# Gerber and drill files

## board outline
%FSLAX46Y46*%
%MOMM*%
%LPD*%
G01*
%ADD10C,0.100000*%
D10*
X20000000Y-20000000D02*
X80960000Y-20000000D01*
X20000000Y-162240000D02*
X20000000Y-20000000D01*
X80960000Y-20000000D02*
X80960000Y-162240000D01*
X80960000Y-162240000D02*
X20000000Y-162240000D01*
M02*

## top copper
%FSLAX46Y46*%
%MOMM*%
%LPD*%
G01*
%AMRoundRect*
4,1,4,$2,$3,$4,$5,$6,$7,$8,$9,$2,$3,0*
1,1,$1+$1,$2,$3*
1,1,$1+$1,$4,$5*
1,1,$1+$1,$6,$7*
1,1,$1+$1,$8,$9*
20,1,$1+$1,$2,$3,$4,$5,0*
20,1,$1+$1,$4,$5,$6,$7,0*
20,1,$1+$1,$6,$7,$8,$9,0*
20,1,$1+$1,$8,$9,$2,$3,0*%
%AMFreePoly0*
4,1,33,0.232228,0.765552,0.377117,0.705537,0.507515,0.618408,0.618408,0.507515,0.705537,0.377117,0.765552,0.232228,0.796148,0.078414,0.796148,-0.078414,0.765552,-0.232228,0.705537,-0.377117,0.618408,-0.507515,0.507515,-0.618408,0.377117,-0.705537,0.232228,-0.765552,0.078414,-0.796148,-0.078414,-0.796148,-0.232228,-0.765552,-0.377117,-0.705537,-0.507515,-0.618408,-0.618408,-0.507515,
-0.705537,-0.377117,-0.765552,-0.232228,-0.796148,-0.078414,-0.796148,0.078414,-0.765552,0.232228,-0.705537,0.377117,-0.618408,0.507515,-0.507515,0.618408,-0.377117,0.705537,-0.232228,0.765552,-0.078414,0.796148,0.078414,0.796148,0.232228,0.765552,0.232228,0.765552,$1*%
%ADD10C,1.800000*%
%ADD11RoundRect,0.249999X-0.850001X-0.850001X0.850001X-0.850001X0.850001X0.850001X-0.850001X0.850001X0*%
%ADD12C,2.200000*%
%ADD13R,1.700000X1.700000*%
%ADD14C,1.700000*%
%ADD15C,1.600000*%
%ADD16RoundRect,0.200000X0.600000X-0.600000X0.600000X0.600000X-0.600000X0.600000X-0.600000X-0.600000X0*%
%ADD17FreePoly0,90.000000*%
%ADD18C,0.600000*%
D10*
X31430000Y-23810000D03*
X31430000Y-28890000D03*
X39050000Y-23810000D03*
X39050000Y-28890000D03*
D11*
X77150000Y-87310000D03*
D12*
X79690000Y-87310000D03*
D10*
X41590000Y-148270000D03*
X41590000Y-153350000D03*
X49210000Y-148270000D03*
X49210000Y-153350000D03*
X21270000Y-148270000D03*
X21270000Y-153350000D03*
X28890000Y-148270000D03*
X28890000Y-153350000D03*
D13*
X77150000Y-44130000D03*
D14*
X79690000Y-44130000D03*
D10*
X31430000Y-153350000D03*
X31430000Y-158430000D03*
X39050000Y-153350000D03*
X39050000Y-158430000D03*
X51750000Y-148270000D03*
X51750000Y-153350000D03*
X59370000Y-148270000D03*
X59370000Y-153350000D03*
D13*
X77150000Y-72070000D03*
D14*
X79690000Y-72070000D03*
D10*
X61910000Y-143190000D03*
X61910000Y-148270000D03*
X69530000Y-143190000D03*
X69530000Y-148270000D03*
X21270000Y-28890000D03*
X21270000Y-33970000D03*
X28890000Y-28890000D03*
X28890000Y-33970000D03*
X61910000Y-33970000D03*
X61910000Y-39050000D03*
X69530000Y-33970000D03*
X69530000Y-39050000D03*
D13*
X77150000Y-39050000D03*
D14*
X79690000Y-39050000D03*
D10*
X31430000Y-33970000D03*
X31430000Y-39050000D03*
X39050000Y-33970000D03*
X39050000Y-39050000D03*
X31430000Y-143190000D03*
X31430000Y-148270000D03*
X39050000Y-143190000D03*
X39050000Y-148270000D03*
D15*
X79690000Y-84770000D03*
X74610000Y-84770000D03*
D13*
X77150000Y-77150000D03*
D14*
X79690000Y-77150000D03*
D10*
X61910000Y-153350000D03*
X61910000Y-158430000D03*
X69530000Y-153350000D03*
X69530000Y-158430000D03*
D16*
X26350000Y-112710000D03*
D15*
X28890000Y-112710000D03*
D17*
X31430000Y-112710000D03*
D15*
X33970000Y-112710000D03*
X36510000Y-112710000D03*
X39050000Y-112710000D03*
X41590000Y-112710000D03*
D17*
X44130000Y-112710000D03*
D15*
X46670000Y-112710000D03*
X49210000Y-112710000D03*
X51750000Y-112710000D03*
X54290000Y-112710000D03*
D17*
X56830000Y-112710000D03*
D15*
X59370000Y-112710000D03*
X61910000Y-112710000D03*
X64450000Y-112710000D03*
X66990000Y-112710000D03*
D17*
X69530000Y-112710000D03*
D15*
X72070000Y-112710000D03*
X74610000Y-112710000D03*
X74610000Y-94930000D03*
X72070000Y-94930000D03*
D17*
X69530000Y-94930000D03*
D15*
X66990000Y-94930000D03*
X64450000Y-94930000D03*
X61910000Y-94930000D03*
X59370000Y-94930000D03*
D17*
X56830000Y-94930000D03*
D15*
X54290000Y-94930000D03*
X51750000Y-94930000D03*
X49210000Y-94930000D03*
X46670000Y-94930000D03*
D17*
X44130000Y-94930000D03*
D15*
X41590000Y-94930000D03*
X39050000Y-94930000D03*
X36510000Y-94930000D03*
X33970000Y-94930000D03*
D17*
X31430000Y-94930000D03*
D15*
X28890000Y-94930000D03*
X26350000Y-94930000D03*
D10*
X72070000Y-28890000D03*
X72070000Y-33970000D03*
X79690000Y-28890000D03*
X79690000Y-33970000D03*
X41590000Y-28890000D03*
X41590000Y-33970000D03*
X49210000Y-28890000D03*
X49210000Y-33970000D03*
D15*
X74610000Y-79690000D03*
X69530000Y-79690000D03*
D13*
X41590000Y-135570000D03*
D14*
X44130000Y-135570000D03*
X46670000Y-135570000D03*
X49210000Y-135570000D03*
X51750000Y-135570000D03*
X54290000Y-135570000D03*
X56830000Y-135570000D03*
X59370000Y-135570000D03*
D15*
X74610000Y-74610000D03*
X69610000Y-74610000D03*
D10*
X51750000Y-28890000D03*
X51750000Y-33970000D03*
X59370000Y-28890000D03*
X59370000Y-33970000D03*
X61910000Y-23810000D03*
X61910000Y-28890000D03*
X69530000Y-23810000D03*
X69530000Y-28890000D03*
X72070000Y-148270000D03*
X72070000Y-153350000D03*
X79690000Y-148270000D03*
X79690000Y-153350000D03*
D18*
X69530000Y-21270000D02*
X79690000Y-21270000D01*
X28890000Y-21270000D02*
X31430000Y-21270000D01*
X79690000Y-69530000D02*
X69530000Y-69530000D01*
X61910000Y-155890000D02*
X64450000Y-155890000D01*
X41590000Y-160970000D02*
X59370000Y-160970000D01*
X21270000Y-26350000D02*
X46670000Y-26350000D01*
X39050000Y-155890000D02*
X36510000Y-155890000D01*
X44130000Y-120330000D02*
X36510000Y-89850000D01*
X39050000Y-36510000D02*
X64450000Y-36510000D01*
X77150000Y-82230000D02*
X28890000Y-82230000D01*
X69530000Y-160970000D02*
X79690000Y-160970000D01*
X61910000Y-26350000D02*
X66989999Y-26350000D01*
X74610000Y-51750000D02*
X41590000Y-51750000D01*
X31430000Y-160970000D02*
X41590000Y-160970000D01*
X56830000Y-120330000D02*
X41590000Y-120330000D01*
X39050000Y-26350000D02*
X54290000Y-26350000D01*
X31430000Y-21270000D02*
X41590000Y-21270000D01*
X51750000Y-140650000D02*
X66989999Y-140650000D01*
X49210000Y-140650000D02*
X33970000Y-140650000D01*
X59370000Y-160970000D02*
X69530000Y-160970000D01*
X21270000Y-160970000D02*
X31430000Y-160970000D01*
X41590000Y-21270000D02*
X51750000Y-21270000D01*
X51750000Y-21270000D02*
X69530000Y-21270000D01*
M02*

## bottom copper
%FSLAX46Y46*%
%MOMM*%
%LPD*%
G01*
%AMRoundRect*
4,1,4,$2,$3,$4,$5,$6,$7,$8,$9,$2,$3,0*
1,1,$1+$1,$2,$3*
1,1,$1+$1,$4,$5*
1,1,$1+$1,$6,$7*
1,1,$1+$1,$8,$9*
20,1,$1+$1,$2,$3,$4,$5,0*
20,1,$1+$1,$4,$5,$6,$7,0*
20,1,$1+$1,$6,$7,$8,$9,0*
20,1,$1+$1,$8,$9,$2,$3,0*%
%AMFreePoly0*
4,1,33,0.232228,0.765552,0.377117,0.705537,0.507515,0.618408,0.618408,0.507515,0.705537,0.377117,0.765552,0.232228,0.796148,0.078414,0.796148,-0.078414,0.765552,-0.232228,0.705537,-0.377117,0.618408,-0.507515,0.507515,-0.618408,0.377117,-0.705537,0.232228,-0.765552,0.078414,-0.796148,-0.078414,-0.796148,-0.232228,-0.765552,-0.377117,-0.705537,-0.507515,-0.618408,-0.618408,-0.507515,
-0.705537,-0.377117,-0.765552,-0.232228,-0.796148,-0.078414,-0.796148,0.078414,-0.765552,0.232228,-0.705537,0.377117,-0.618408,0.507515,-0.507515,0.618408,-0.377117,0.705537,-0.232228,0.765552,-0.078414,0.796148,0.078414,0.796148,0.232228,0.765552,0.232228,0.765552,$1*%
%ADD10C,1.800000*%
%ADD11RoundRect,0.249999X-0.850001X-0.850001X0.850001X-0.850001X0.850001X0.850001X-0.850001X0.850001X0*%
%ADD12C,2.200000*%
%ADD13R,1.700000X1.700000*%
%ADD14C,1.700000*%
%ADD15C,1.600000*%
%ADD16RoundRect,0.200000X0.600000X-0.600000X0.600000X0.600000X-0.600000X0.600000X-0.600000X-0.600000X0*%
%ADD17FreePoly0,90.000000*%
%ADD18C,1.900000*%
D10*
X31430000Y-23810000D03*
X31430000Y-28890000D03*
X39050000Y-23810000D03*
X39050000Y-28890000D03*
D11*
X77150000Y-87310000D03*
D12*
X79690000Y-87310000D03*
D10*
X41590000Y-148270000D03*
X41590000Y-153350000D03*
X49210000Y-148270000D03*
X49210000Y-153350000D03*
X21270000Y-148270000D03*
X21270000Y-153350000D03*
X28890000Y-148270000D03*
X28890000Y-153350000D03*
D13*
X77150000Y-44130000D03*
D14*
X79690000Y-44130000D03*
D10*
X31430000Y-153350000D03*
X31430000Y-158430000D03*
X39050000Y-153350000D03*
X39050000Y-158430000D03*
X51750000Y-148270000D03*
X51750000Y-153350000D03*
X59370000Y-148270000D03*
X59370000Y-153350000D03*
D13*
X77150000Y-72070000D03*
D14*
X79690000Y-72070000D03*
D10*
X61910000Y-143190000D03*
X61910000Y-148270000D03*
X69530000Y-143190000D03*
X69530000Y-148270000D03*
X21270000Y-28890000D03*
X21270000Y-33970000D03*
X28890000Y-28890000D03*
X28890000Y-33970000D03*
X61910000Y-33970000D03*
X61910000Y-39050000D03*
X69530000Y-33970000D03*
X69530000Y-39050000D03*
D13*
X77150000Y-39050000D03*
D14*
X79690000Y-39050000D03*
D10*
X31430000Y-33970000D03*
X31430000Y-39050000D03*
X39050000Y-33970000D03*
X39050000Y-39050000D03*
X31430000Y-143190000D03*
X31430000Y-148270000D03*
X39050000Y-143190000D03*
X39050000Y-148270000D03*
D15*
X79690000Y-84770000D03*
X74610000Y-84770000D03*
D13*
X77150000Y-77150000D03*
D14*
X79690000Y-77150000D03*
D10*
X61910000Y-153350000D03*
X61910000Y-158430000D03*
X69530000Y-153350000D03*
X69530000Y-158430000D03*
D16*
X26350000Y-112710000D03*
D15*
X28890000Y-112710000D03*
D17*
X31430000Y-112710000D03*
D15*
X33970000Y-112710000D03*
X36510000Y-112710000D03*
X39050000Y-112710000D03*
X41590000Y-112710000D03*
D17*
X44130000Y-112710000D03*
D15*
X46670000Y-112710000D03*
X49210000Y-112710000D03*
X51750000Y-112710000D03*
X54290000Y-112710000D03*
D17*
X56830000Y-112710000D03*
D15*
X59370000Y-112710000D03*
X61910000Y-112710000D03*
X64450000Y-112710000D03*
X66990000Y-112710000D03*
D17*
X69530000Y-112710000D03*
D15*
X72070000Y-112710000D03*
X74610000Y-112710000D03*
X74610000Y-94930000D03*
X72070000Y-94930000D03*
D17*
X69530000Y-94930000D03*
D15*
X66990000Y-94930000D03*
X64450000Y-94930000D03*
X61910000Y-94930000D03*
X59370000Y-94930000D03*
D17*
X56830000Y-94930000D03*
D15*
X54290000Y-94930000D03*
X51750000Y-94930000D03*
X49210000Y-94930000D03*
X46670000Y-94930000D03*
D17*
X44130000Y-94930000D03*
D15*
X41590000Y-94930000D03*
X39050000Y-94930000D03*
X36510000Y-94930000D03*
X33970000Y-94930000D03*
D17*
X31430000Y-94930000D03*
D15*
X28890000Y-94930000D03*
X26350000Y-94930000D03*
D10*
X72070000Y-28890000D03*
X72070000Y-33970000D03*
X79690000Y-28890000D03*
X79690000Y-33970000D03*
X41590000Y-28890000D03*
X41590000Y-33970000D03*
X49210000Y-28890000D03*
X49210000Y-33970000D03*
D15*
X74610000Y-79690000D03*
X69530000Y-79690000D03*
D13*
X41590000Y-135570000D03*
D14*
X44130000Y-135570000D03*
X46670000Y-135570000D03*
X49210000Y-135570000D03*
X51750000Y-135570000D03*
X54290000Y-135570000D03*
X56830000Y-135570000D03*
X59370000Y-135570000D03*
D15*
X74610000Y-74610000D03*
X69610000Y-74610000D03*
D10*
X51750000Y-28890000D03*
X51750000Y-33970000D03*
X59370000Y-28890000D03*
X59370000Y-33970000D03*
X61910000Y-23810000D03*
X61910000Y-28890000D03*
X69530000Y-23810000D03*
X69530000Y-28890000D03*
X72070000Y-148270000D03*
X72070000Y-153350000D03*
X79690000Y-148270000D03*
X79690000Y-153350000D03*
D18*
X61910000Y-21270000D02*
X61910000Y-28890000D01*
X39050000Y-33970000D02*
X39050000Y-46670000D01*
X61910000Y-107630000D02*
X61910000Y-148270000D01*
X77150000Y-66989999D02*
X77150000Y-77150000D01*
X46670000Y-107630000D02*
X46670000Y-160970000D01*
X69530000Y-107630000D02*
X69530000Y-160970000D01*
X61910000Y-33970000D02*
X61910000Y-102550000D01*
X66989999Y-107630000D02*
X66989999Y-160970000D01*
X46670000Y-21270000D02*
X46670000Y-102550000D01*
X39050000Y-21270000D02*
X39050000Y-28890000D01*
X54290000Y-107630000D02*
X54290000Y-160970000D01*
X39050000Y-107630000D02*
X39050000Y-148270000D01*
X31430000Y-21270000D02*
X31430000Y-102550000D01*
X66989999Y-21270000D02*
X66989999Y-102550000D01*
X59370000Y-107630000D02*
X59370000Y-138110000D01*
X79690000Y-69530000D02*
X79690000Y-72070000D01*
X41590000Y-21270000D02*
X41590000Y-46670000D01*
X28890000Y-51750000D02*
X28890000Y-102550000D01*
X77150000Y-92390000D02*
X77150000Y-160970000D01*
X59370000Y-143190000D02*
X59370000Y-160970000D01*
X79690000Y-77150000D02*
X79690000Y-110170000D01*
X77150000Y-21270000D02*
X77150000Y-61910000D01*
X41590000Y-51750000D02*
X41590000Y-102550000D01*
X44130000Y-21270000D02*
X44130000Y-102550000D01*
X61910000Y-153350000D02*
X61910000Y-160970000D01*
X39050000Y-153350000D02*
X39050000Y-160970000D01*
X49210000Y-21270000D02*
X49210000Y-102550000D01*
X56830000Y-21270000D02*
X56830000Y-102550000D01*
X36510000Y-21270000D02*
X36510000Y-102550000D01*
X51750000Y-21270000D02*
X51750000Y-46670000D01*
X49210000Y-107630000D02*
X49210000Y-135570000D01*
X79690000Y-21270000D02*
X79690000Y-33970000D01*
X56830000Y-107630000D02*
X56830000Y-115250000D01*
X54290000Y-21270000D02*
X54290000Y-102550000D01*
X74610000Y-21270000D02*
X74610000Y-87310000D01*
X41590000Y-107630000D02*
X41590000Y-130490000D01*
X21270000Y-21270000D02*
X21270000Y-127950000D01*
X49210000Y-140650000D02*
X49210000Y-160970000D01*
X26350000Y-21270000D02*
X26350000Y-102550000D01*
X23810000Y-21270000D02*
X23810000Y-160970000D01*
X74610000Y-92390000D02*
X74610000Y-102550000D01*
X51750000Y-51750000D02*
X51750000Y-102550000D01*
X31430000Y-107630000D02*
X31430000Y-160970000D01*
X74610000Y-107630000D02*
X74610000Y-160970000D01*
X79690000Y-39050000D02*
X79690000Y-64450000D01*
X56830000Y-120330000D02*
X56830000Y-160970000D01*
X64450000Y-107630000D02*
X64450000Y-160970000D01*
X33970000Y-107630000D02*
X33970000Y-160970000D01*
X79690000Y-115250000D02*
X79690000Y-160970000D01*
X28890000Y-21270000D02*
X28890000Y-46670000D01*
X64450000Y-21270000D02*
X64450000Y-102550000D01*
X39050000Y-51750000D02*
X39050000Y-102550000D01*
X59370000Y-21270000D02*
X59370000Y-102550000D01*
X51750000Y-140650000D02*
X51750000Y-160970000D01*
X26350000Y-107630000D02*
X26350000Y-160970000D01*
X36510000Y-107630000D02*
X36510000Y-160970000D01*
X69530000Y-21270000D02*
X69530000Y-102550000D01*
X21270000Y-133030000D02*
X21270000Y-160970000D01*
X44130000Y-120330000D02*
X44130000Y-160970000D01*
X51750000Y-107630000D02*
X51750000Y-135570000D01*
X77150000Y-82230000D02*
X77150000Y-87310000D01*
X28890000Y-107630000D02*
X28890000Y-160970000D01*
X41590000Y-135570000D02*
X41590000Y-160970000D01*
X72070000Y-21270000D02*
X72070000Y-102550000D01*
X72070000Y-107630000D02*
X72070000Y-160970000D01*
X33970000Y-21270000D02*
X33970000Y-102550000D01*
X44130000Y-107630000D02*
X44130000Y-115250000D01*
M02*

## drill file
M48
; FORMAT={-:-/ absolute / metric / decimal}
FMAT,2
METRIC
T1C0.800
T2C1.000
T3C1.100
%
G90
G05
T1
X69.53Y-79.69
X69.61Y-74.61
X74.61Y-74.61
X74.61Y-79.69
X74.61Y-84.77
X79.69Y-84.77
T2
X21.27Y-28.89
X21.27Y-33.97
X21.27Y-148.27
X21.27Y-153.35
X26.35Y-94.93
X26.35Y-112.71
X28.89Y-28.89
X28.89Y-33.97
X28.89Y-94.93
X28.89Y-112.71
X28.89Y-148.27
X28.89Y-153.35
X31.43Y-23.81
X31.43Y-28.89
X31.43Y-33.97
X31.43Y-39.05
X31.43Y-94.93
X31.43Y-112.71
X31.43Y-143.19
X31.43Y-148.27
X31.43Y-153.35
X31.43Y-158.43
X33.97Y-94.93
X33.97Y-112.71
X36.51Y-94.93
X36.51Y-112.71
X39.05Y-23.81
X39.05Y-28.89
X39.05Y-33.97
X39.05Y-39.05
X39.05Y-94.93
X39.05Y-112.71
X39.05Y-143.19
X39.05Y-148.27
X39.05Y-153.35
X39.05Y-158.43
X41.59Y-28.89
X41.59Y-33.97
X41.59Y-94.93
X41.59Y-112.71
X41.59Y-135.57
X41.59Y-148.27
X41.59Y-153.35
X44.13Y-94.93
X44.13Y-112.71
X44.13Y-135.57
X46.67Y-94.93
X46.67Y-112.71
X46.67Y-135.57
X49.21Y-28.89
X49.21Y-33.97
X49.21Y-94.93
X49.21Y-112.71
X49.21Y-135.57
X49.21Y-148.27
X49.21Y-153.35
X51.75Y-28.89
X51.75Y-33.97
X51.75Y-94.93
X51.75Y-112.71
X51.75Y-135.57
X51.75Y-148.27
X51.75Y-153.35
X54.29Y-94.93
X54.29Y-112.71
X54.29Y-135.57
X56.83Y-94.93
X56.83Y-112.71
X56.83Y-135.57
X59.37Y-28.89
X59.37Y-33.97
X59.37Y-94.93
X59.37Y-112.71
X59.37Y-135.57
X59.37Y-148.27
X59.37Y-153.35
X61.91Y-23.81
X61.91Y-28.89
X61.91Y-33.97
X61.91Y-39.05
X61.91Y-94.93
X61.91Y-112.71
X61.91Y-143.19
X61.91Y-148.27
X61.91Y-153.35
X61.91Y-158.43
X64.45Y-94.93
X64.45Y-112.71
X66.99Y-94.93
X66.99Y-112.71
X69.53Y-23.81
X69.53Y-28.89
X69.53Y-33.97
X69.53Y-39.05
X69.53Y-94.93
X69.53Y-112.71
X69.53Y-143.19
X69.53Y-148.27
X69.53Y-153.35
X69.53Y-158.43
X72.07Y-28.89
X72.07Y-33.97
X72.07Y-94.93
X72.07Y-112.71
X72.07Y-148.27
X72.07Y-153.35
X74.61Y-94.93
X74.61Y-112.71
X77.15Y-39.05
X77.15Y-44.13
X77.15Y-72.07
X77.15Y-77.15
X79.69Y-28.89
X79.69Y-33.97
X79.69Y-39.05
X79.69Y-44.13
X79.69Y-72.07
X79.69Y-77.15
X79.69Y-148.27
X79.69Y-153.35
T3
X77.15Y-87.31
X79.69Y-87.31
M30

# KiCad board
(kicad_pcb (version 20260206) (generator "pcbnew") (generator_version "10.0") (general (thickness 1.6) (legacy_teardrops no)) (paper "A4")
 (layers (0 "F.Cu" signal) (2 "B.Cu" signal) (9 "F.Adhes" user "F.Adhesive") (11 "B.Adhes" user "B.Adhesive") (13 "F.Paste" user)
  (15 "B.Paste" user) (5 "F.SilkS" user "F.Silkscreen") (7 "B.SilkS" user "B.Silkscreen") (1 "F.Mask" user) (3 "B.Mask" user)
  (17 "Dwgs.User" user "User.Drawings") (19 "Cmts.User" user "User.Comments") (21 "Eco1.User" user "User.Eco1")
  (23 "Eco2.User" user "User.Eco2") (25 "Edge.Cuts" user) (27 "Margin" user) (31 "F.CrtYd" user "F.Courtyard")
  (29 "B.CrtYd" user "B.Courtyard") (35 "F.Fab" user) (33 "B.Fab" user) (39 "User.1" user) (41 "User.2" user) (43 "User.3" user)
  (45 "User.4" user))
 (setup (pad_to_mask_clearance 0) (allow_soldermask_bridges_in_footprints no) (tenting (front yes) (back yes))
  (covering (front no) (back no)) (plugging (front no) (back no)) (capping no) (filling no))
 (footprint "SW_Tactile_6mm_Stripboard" (layer "F.Cu") (at 31.43 23.81)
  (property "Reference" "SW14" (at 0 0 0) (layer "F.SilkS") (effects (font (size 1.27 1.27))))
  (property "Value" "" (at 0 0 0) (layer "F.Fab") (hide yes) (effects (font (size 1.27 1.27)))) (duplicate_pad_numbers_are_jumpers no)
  (pad "1" thru_hole circle (at 0 0) (size 1.8 1.8) (drill 1) (layers "*.Cu" "*.Mask") (remove_unused_layers no))
  (pad "1" thru_hole circle (at 0 5.08) (size 1.8 1.8) (drill 1) (layers "*.Cu" "*.Mask") (remove_unused_layers no))
  (pad "2" thru_hole circle (at 7.62 0) (size 1.8 1.8) (drill 1) (layers "*.Cu" "*.Mask") (remove_unused_layers no))
  (pad "2" thru_hole circle (at 7.62 5.08) (size 1.8 1.8) (drill 1) (layers "*.Cu" "*.Mask") (remove_unused_layers no)))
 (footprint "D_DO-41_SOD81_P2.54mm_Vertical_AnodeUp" (layer "F.Cu") (at 77.15 87.31)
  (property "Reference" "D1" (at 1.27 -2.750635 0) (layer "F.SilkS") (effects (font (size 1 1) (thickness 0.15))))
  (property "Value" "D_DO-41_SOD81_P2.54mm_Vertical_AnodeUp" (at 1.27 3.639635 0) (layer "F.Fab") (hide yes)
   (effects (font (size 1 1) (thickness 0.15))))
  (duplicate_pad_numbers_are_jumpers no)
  (pad "1" thru_hole roundrect (at 0 0) (size 2.2 2.2) (drill 1.1) (layers "*.Cu" "*.Mask") (remove_unused_layers no)
   (roundrect_rratio 0.113636))
  (pad "2" thru_hole circle (at 2.54 0) (size 2.2 2.2) (drill 1.1) (layers "*.Cu" "*.Mask") (remove_unused_layers no)))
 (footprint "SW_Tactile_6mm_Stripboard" (layer "F.Cu") (at 41.59 148.27)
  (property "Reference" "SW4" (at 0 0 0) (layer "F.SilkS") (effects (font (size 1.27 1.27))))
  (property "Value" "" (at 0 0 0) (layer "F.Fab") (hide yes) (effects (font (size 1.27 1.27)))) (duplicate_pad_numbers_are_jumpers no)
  (pad "1" thru_hole circle (at 0 0) (size 1.8 1.8) (drill 1) (layers "*.Cu" "*.Mask") (remove_unused_layers no))
  (pad "1" thru_hole circle (at 0 5.08) (size 1.8 1.8) (drill 1) (layers "*.Cu" "*.Mask") (remove_unused_layers no))
  (pad "2" thru_hole circle (at 7.62 0) (size 1.8 1.8) (drill 1) (layers "*.Cu" "*.Mask") (remove_unused_layers no))
  (pad "2" thru_hole circle (at 7.62 5.08) (size 1.8 1.8) (drill 1) (layers "*.Cu" "*.Mask") (remove_unused_layers no)))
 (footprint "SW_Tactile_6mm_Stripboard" (layer "F.Cu") (at 21.27 148.27)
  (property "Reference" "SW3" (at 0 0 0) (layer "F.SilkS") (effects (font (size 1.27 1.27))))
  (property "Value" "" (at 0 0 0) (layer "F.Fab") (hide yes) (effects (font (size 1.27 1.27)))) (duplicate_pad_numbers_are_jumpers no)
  (pad "1" thru_hole circle (at 0 0) (size 1.8 1.8) (drill 1) (layers "*.Cu" "*.Mask") (remove_unused_layers no))
  (pad "1" thru_hole circle (at 0 5.08) (size 1.8 1.8) (drill 1) (layers "*.Cu" "*.Mask") (remove_unused_layers no))
  (pad "2" thru_hole circle (at 7.62 0) (size 1.8 1.8) (drill 1) (layers "*.Cu" "*.Mask") (remove_unused_layers no))
  (pad "2" thru_hole circle (at 7.62 5.08) (size 1.8 1.8) (drill 1) (layers "*.Cu" "*.Mask") (remove_unused_layers no)))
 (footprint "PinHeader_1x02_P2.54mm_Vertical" (layer "F.Cu") (at 77.15 44.13 90)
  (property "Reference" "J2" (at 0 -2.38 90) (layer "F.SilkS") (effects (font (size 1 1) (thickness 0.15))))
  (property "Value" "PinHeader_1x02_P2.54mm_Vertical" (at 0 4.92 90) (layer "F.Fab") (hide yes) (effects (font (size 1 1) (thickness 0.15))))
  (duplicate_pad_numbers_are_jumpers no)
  (pad "1" thru_hole rect (at 0 0 90) (size 1.7 1.7) (drill 1) (layers "*.Cu" "*.Mask") (remove_unused_layers no))
  (pad "2" thru_hole circle (at 0 2.54 90) (size 1.7 1.7) (drill 1) (layers "*.Cu" "*.Mask") (remove_unused_layers no)))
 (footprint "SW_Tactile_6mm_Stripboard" (layer "F.Cu") (at 31.43 153.35)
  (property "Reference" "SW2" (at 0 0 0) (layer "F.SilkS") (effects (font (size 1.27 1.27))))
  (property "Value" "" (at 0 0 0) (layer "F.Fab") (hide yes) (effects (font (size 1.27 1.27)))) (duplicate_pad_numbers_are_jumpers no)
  (pad "1" thru_hole circle (at 0 0) (size 1.8 1.8) (drill 1) (layers "*.Cu" "*.Mask") (remove_unused_layers no))
  (pad "1" thru_hole circle (at 0 5.08) (size 1.8 1.8) (drill 1) (layers "*.Cu" "*.Mask") (remove_unused_layers no))
  (pad "2" thru_hole circle (at 7.62 0) (size 1.8 1.8) (drill 1) (layers "*.Cu" "*.Mask") (remove_unused_layers no))
  (pad "2" thru_hole circle (at 7.62 5.08) (size 1.8 1.8) (drill 1) (layers "*.Cu" "*.Mask") (remove_unused_layers no)))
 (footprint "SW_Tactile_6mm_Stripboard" (layer "F.Cu") (at 51.75 148.27)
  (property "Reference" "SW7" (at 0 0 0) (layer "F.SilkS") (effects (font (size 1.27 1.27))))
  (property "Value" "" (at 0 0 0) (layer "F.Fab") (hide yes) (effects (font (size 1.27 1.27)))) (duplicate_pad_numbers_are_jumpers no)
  (pad "1" thru_hole circle (at 0 0) (size 1.8 1.8) (drill 1) (layers "*.Cu" "*.Mask") (remove_unused_layers no))
  (pad "1" thru_hole circle (at 0 5.08) (size 1.8 1.8) (drill 1) (layers "*.Cu" "*.Mask") (remove_unused_layers no))
  (pad "2" thru_hole circle (at 7.62 0) (size 1.8 1.8) (drill 1) (layers "*.Cu" "*.Mask") (remove_unused_layers no))
  (pad "2" thru_hole circle (at 7.62 5.08) (size 1.8 1.8) (drill 1) (layers "*.Cu" "*.Mask") (remove_unused_layers no)))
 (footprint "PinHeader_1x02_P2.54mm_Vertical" (layer "F.Cu") (at 77.15 72.07 90)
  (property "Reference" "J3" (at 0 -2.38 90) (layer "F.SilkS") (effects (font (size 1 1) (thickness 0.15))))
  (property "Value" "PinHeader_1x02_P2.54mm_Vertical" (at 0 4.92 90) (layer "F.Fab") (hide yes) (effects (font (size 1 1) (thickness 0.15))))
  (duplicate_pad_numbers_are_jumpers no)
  (pad "1" thru_hole rect (at 0 0 90) (size 1.7 1.7) (drill 1) (layers "*.Cu" "*.Mask") (remove_unused_layers no))
  (pad "2" thru_hole circle (at 0 2.54 90) (size 1.7 1.7) (drill 1) (layers "*.Cu" "*.Mask") (remove_unused_layers no)))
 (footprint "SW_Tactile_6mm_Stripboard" (layer "F.Cu") (at 61.91 143.19)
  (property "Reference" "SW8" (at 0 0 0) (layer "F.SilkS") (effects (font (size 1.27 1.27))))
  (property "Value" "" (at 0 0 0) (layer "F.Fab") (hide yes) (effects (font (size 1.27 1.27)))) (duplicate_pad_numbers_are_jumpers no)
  (pad "1" thru_hole circle (at 0 0) (size 1.8 1.8) (drill 1) (layers "*.Cu" "*.Mask") (remove_unused_layers no))
  (pad "1" thru_hole circle (at 0 5.08) (size 1.8 1.8) (drill 1) (layers "*.Cu" "*.Mask") (remove_unused_layers no))
  (pad "2" thru_hole circle (at 7.62 0) (size 1.8 1.8) (drill 1) (layers "*.Cu" "*.Mask") (remove_unused_layers no))
  (pad "2" thru_hole circle (at 7.62 5.08) (size 1.8 1.8) (drill 1) (layers "*.Cu" "*.Mask") (remove_unused_layers no)))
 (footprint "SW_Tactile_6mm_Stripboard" (layer "F.Cu") (at 21.27 28.89)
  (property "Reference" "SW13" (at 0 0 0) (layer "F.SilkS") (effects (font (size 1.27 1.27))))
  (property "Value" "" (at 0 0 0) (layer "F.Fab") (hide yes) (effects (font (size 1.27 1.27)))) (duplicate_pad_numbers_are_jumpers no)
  (pad "1" thru_hole circle (at 0 0) (size 1.8 1.8) (drill 1) (layers "*.Cu" "*.Mask") (remove_unused_layers no))
  (pad "1" thru_hole circle (at 0 5.08) (size 1.8 1.8) (drill 1) (layers "*.Cu" "*.Mask") (remove_unused_layers no))
  (pad "2" thru_hole circle (at 7.62 0) (size 1.8 1.8) (drill 1) (layers "*.Cu" "*.Mask") (remove_unused_layers no))
  (pad "2" thru_hole circle (at 7.62 5.08) (size 1.8 1.8) (drill 1) (layers "*.Cu" "*.Mask") (remove_unused_layers no)))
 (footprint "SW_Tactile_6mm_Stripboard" (layer "F.Cu") (at 61.91 33.97)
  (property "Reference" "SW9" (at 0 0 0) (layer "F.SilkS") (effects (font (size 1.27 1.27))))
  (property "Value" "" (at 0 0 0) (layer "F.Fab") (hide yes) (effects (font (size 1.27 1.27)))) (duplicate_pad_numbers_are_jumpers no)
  (pad "1" thru_hole circle (at 0 0) (size 1.8 1.8) (drill 1) (layers "*.Cu" "*.Mask") (remove_unused_layers no))
  (pad "1" thru_hole circle (at 0 5.08) (size 1.8 1.8) (drill 1) (layers "*.Cu" "*.Mask") (remove_unused_layers no))
  (pad "2" thru_hole circle (at 7.62 0) (size 1.8 1.8) (drill 1) (layers "*.Cu" "*.Mask") (remove_unused_layers no))
  (pad "2" thru_hole circle (at 7.62 5.08) (size 1.8 1.8) (drill 1) (layers "*.Cu" "*.Mask") (remove_unused_layers no)))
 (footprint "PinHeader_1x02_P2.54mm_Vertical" (layer "F.Cu") (at 77.15 39.05 90)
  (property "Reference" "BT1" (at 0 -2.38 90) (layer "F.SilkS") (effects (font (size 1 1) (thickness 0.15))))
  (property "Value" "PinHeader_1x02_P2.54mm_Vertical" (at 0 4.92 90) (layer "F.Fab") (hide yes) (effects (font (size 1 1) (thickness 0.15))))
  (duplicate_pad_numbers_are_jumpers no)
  (pad "1" thru_hole rect (at 0 0 90) (size 1.7 1.7) (drill 1) (layers "*.Cu" "*.Mask") (remove_unused_layers no))
  (pad "2" thru_hole circle (at 0 2.54 90) (size 1.7 1.7) (drill 1) (layers "*.Cu" "*.Mask") (remove_unused_layers no)))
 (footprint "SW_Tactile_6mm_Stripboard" (layer "F.Cu") (at 31.43 33.97)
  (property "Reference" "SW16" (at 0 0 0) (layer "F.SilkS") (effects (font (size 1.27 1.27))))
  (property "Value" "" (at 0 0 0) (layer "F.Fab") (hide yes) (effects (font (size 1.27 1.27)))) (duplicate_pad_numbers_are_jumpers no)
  (pad "1" thru_hole circle (at 0 0) (size 1.8 1.8) (drill 1) (layers "*.Cu" "*.Mask") (remove_unused_layers no))
  (pad "1" thru_hole circle (at 0 5.08) (size 1.8 1.8) (drill 1) (layers "*.Cu" "*.Mask") (remove_unused_layers no))
  (pad "2" thru_hole circle (at 7.62 0) (size 1.8 1.8) (drill 1) (layers "*.Cu" "*.Mask") (remove_unused_layers no))
  (pad "2" thru_hole circle (at 7.62 5.08) (size 1.8 1.8) (drill 1) (layers "*.Cu" "*.Mask") (remove_unused_layers no)))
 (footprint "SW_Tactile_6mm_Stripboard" (layer "F.Cu") (at 31.43 143.19)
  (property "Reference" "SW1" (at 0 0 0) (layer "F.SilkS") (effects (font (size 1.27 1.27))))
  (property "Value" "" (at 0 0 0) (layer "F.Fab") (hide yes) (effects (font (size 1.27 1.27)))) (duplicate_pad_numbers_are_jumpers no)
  (pad "1" thru_hole circle (at 0 0) (size 1.8 1.8) (drill 1) (layers "*.Cu" "*.Mask") (remove_unused_layers no))
  (pad "1" thru_hole circle (at 0 5.08) (size 1.8 1.8) (drill 1) (layers "*.Cu" "*.Mask") (remove_unused_layers no))
  (pad "2" thru_hole circle (at 7.62 0) (size 1.8 1.8) (drill 1) (layers "*.Cu" "*.Mask") (remove_unused_layers no))
  (pad "2" thru_hole circle (at 7.62 5.08) (size 1.8 1.8) (drill 1) (layers "*.Cu" "*.Mask") (remove_unused_layers no)))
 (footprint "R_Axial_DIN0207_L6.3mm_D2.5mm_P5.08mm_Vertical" (layer "F.Cu") (at 79.69 84.77 180)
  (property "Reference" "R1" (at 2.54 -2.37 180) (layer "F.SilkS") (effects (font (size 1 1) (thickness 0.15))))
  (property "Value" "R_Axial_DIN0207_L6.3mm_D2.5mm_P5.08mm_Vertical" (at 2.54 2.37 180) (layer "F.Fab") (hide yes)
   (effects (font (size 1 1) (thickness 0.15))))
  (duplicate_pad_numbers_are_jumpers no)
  (pad "1" thru_hole circle (at 0 0 180) (size 1.6 1.6) (drill 0.8) (layers "*.Cu" "*.Mask") (remove_unused_layers no))
  (pad "2" thru_hole circle (at 5.08 0 180) (size 1.6 1.6) (drill 0.8) (layers "*.Cu" "*.Mask") (remove_unused_layers no)))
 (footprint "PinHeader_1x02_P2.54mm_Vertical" (layer "F.Cu") (at 77.15 77.15 90)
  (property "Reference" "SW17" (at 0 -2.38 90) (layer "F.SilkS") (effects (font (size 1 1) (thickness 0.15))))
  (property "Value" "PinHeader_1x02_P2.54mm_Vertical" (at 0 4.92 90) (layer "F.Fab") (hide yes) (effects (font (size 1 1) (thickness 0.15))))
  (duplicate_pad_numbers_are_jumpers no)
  (pad "1" thru_hole rect (at 0 0 90) (size 1.7 1.7) (drill 1) (layers "*.Cu" "*.Mask") (remove_unused_layers no))
  (pad "2" thru_hole circle (at 0 2.54 90) (size 1.7 1.7) (drill 1) (layers "*.Cu" "*.Mask") (remove_unused_layers no)))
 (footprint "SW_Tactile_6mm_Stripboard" (layer "F.Cu") (at 61.91 153.35)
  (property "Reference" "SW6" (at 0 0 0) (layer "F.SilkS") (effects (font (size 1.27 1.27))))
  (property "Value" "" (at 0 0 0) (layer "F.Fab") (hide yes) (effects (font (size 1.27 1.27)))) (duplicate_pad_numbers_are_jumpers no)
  (pad "1" thru_hole circle (at 0 0) (size 1.8 1.8) (drill 1) (layers "*.Cu" "*.Mask") (remove_unused_layers no))
  (pad "1" thru_hole circle (at 0 5.08) (size 1.8 1.8) (drill 1) (layers "*.Cu" "*.Mask") (remove_unused_layers no))
  (pad "2" thru_hole circle (at 7.62 0) (size 1.8 1.8) (drill 1) (layers "*.Cu" "*.Mask") (remove_unused_layers no))
  (pad "2" thru_hole circle (at 7.62 5.08) (size 1.8 1.8) (drill 1) (layers "*.Cu" "*.Mask") (remove_unused_layers no)))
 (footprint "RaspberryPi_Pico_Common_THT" (layer "F.Cu") (at 26.35 112.71 90)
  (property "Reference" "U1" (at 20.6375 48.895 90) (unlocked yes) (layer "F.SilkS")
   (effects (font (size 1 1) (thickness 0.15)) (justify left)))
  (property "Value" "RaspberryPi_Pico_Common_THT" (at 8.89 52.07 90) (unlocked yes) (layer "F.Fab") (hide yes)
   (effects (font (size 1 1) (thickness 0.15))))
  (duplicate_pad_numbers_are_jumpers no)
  (pad "1" thru_hole roundrect (at 0 0 90) (size 1.6 1.6) (drill 1) (layers "*.Cu" "*.Mask") (remove_unused_layers no)
   (roundrect_rratio 0.125))
  (pad "2" thru_hole circle (at 0 2.54 90) (size 1.6 1.6) (drill 1) (layers "*.Cu" "*.Mask") (remove_unused_layers no))
  (pad "3" thru_hole custom (at 0 5.08 90) (size 1.6 1.6) (drill 1) (layers "*.Cu" "*.Mask") (remove_unused_layers no)
   (options (clearance outline) (anchor circle)) (primitives))
  (pad "4" thru_hole circle (at 0 7.62 90) (size 1.6 1.6) (drill 1) (layers "*.Cu" "*.Mask") (remove_unused_layers no))
  (pad "5" thru_hole circle (at 0 10.16 90) (size 1.6 1.6) (drill 1) (layers "*.Cu" "*.Mask") (remove_unused_layers no))
  (pad "6" thru_hole circle (at 0 12.7 90) (size 1.6 1.6) (drill 1) (layers "*.Cu" "*.Mask") (remove_unused_layers no))
  (pad "7" thru_hole circle (at 0 15.24 90) (size 1.6 1.6) (drill 1) (layers "*.Cu" "*.Mask") (remove_unused_layers no))
  (pad "8" thru_hole custom (at 0 17.78 90) (size 1.6 1.6) (drill 1) (layers "*.Cu" "*.Mask") (remove_unused_layers no)
   (options (clearance outline) (anchor circle)) (primitives))
  (pad "9" thru_hole circle (at 0 20.32 90) (size 1.6 1.6) (drill 1) (layers "*.Cu" "*.Mask") (remove_unused_layers no))
  (pad "10" thru_hole circle (at 0 22.86 90) (size 1.6 1.6) (drill 1) (layers "*.Cu" "*.Mask") (remove_unused_layers no))
  (pad "11" thru_hole circle (at 0 25.4 90) (size 1.6 1.6) (drill 1) (layers "*.Cu" "*.Mask") (remove_unused_layers no))
  (pad "12" thru_hole circle (at 0 27.94 90) (size 1.6 1.6) (drill 1) (layers "*.Cu" "*.Mask") (remove_unused_layers no))
  (pad "13" thru_hole custom (at 0 30.48 90) (size 1.6 1.6) (drill 1) (layers "*.Cu" "*.Mask") (remove_unused_layers no)
   (options (clearance outline) (anchor circle)) (primitives))
  (pad "14" thru_hole circle (at 0 33.02 90) (size 1.6 1.6) (drill 1) (layers "*.Cu" "*.Mask") (remove_unused_layers no))
  (pad "15" thru_hole circle (at 0 35.56 90) (size 1.6 1.6) (drill 1) (layers "*.Cu" "*.Mask") (remove_unused_layers no))
  (pad "16" thru_hole circle (at 0 38.1 90) (size 1.6 1.6) (drill 1) (layers "*.Cu" "*.Mask") (remove_unused_layers no))
  (pad "17" thru_hole circle (at 0 40.64 90) (size 1.6 1.6) (drill 1) (layers "*.Cu" "*.Mask") (remove_unused_layers no))
  (pad "18" thru_hole custom (at 0 43.18 90) (size 1.6 1.6) (drill 1) (layers "*.Cu" "*.Mask") (remove_unused_layers no)
   (options (clearance outline) (anchor circle)) (primitives))
  (pad "19" thru_hole circle (at 0 45.72 90) (size 1.6 1.6) (drill 1) (layers "*.Cu" "*.Mask") (remove_unused_layers no))
  (pad "20" thru_hole circle (at 0 48.26 90) (size 1.6 1.6) (drill 1) (layers "*.Cu" "*.Mask") (remove_unused_layers no))
  (pad "21" thru_hole circle (at 17.78 48.26 90) (size 1.6 1.6) (drill 1) (layers "*.Cu" "*.Mask") (remove_unused_layers no))
  (pad "22" thru_hole circle (at 17.78 45.72 90) (size 1.6 1.6) (drill 1) (layers "*.Cu" "*.Mask") (remove_unused_layers no))
  (pad "23" thru_hole custom (at 17.78 43.18 90) (size 1.6 1.6) (drill 1) (layers "*.Cu" "*.Mask") (remove_unused_layers no)
   (options (clearance outline) (anchor circle)) (primitives))
  (pad "24" thru_hole circle (at 17.78 40.64 90) (size 1.6 1.6) (drill 1) (layers "*.Cu" "*.Mask") (remove_unused_layers no))
  (pad "25" thru_hole circle (at 17.78 38.1 90) (size 1.6 1.6) (drill 1) (layers "*.Cu" "*.Mask") (remove_unused_layers no))
  (pad "26" thru_hole circle (at 17.78 35.56 90) (size 1.6 1.6) (drill 1) (layers "*.Cu" "*.Mask") (remove_unused_layers no))
  (pad "27" thru_hole circle (at 17.78 33.02 90) (size 1.6 1.6) (drill 1) (layers "*.Cu" "*.Mask") (remove_unused_layers no))
  (pad "28" thru_hole custom (at 17.78 30.48 90) (size 1.6 1.6) (drill 1) (layers "*.Cu" "*.Mask") (remove_unused_layers no)
   (options (clearance outline) (anchor circle)) (primitives))
  (pad "29" thru_hole circle (at 17.78 27.94 90) (size 1.6 1.6) (drill 1) (layers "*.Cu" "*.Mask") (remove_unused_layers no))
  (pad "30" thru_hole circle (at 17.78 25.4 90) (size 1.6 1.6) (drill 1) (layers "*.Cu" "*.Mask") (remove_unused_layers no))
  (pad "31" thru_hole circle (at 17.78 22.86 90) (size 1.6 1.6) (drill 1) (layers "*.Cu" "*.Mask") (remove_unused_layers no))
  (pad "32" thru_hole circle (at 17.78 20.32 90) (size 1.6 1.6) (drill 1) (layers "*.Cu" "*.Mask") (remove_unused_layers no))
  (pad "33" thru_hole custom (at 17.78 17.78 90) (size 1.6 1.6) (drill 1) (layers "*.Cu" "*.Mask") (remove_unused_layers no)
   (options (clearance outline) (anchor circle)) (primitives))
  (pad "34" thru_hole circle (at 17.78 15.24 90) (size 1.6 1.6) (drill 1) (layers "*.Cu" "*.Mask") (remove_unused_layers no))
  (pad "35" thru_hole circle (at 17.78 12.7 90) (size 1.6 1.6) (drill 1) (layers "*.Cu" "*.Mask") (remove_unused_layers no))
  (pad "36" thru_hole circle (at 17.78 10.16 90) (size 1.6 1.6) (drill 1) (layers "*.Cu" "*.Mask") (remove_unused_layers no))
  (pad "37" thru_hole circle (at 17.78 7.62 90) (size 1.6 1.6) (drill 1) (layers "*.Cu" "*.Mask") (remove_unused_layers no))
  (pad "38" thru_hole custom (at 17.78 5.08 90) (size 1.6 1.6) (drill 1) (layers "*.Cu" "*.Mask") (remove_unused_layers no)
   (options (clearance outline) (anchor circle)) (primitives))
  (pad "39" thru_hole circle (at 17.78 2.54 90) (size 1.6 1.6) (drill 1) (layers "*.Cu" "*.Mask") (remove_unused_layers no))
  (pad "40" thru_hole circle (at 17.78 0 90) (size 1.6 1.6) (drill 1) (layers "*.Cu" "*.Mask") (remove_unused_layers no))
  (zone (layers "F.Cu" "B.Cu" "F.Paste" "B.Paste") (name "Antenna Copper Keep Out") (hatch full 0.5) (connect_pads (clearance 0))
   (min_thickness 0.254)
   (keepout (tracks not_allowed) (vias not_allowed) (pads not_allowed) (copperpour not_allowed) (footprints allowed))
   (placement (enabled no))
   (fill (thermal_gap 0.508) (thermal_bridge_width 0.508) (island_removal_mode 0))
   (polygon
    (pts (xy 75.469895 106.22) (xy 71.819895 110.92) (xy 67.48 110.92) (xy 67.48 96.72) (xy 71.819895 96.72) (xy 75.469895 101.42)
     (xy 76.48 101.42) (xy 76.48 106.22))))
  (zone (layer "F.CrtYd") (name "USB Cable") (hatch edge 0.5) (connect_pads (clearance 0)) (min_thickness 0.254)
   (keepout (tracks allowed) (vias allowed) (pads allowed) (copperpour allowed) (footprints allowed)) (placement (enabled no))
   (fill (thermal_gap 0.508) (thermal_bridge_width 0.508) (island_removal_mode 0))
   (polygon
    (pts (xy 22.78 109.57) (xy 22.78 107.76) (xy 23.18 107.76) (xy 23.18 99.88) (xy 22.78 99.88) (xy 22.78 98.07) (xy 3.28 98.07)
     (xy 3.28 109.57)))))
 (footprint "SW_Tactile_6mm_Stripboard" (layer "F.Cu") (at 72.07 28.89)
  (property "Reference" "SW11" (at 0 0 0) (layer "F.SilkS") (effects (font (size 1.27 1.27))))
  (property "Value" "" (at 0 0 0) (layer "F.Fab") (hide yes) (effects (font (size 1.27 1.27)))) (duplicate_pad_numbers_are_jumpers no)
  (pad "1" thru_hole circle (at 0 0) (size 1.8 1.8) (drill 1) (layers "*.Cu" "*.Mask") (remove_unused_layers no))
  (pad "1" thru_hole circle (at 0 5.08) (size 1.8 1.8) (drill 1) (layers "*.Cu" "*.Mask") (remove_unused_layers no))
  (pad "2" thru_hole circle (at 7.62 0) (size 1.8 1.8) (drill 1) (layers "*.Cu" "*.Mask") (remove_unused_layers no))
  (pad "2" thru_hole circle (at 7.62 5.08) (size 1.8 1.8) (drill 1) (layers "*.Cu" "*.Mask") (remove_unused_layers no)))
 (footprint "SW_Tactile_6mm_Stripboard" (layer "F.Cu") (at 41.59 28.89)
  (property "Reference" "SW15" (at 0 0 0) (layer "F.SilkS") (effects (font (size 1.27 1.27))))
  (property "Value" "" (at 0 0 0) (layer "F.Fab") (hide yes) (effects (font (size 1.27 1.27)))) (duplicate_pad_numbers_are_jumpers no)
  (pad "1" thru_hole circle (at 0 0) (size 1.8 1.8) (drill 1) (layers "*.Cu" "*.Mask") (remove_unused_layers no))
  (pad "1" thru_hole circle (at 0 5.08) (size 1.8 1.8) (drill 1) (layers "*.Cu" "*.Mask") (remove_unused_layers no))
  (pad "2" thru_hole circle (at 7.62 0) (size 1.8 1.8) (drill 1) (layers "*.Cu" "*.Mask") (remove_unused_layers no))
  (pad "2" thru_hole circle (at 7.62 5.08) (size 1.8 1.8) (drill 1) (layers "*.Cu" "*.Mask") (remove_unused_layers no)))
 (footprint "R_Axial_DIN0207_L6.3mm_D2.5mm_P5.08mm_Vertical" (layer "F.Cu") (at 74.61 79.69 180)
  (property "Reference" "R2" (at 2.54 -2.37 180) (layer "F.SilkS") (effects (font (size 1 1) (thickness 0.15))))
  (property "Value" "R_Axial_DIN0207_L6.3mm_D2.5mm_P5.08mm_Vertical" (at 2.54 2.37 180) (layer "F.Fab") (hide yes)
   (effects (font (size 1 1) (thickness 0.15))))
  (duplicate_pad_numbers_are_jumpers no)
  (pad "1" thru_hole circle (at 0 0 180) (size 1.6 1.6) (drill 0.8) (layers "*.Cu" "*.Mask") (remove_unused_layers no))
  (pad "2" thru_hole circle (at 5.08 0 180) (size 1.6 1.6) (drill 0.8) (layers "*.Cu" "*.Mask") (remove_unused_layers no)))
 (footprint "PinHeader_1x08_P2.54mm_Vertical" (layer "F.Cu") (at 41.59 135.57 90)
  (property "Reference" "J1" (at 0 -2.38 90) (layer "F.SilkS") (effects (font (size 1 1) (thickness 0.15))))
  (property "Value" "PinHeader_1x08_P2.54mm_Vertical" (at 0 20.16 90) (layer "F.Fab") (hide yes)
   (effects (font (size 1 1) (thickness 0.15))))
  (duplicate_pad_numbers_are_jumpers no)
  (pad "1" thru_hole rect (at 0 0 90) (size 1.7 1.7) (drill 1) (layers "*.Cu" "*.Mask") (remove_unused_layers no))
  (pad "2" thru_hole circle (at 0 2.54 90) (size 1.7 1.7) (drill 1) (layers "*.Cu" "*.Mask") (remove_unused_layers no))
  (pad "3" thru_hole circle (at 0 5.08 90) (size 1.7 1.7) (drill 1) (layers "*.Cu" "*.Mask") (remove_unused_layers no))
  (pad "4" thru_hole circle (at 0 7.62 90) (size 1.7 1.7) (drill 1) (layers "*.Cu" "*.Mask") (remove_unused_layers no))
  (pad "5" thru_hole circle (at 0 10.16 90) (size 1.7 1.7) (drill 1) (layers "*.Cu" "*.Mask") (remove_unused_layers no))
  (pad "6" thru_hole circle (at 0 12.7 90) (size 1.7 1.7) (drill 1) (layers "*.Cu" "*.Mask") (remove_unused_layers no))
  (pad "7" thru_hole circle (at 0 15.24 90) (size 1.7 1.7) (drill 1) (layers "*.Cu" "*.Mask") (remove_unused_layers no))
  (pad "8" thru_hole circle (at 0 17.78 90) (size 1.7 1.7) (drill 1) (layers "*.Cu" "*.Mask") (remove_unused_layers no)))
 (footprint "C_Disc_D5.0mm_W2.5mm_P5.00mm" (layer "F.Cu") (at 74.61 74.61 180)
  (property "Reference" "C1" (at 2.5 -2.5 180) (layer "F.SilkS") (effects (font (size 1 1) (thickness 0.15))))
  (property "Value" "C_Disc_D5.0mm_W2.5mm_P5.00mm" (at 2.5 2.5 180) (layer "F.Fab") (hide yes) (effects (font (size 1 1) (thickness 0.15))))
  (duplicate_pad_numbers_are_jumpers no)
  (pad "1" thru_hole circle (at 0 0 180) (size 1.6 1.6) (drill 0.8) (layers "*.Cu" "*.Mask") (remove_unused_layers no))
  (pad "2" thru_hole circle (at 5 0 180) (size 1.6 1.6) (drill 0.8) (layers "*.Cu" "*.Mask") (remove_unused_layers no)))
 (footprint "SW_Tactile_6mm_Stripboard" (layer "F.Cu") (at 51.75 28.89)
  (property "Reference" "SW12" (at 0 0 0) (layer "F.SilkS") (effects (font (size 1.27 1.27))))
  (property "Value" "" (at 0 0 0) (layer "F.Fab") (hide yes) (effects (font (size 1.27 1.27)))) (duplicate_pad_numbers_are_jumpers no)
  (pad "1" thru_hole circle (at 0 0) (size 1.8 1.8) (drill 1) (layers "*.Cu" "*.Mask") (remove_unused_layers no))
  (pad "1" thru_hole circle (at 0 5.08) (size 1.8 1.8) (drill 1) (layers "*.Cu" "*.Mask") (remove_unused_layers no))
  (pad "2" thru_hole circle (at 7.62 0) (size 1.8 1.8) (drill 1) (layers "*.Cu" "*.Mask") (remove_unused_layers no))
  (pad "2" thru_hole circle (at 7.62 5.08) (size 1.8 1.8) (drill 1) (layers "*.Cu" "*.Mask") (remove_unused_layers no)))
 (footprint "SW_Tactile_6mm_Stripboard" (layer "F.Cu") (at 61.91 23.81)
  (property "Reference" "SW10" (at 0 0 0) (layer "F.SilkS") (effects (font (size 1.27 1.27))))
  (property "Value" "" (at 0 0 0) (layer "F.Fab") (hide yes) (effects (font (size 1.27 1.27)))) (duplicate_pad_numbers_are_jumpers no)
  (pad "1" thru_hole circle (at 0 0) (size 1.8 1.8) (drill 1) (layers "*.Cu" "*.Mask") (remove_unused_layers no))
  (pad "1" thru_hole circle (at 0 5.08) (size 1.8 1.8) (drill 1) (layers "*.Cu" "*.Mask") (remove_unused_layers no))
  (pad "2" thru_hole circle (at 7.62 0) (size 1.8 1.8) (drill 1) (layers "*.Cu" "*.Mask") (remove_unused_layers no))
  (pad "2" thru_hole circle (at 7.62 5.08) (size 1.8 1.8) (drill 1) (layers "*.Cu" "*.Mask") (remove_unused_layers no)))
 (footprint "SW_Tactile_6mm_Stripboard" (layer "F.Cu") (at 72.07 148.27)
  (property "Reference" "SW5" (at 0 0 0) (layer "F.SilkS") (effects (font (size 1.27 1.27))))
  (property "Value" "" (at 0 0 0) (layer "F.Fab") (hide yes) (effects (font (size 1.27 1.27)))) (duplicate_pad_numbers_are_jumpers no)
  (pad "1" thru_hole circle (at 0 0) (size 1.8 1.8) (drill 1) (layers "*.Cu" "*.Mask") (remove_unused_layers no))
  (pad "1" thru_hole circle (at 0 5.08) (size 1.8 1.8) (drill 1) (layers "*.Cu" "*.Mask") (remove_unused_layers no))
  (pad "2" thru_hole circle (at 7.62 0) (size 1.8 1.8) (drill 1) (layers "*.Cu" "*.Mask") (remove_unused_layers no))
  (pad "2" thru_hole circle (at 7.62 5.08) (size 1.8 1.8) (drill 1) (layers "*.Cu" "*.Mask") (remove_unused_layers no)))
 (gr_line (start 20 20) (end 80.96 20) (stroke (width 0.1) (type default)) (layer "Edge.Cuts"))
 (gr_line (start 20 162.24) (end 20 20) (stroke (width 0.1) (type default)) (layer "Edge.Cuts"))
 (gr_line (start 80.96 20) (end 80.96 162.24) (stroke (width 0.1) (type default)) (layer "Edge.Cuts"))
 (gr_line (start 80.96 162.24) (end 20 162.24) (stroke (width 0.1) (type default)) (layer "Edge.Cuts"))
 (segment (start 69.53 21.27) (end 79.69 21.27) (width 0.6) (layer "F.Cu") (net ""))
 (segment (start 28.89 21.27) (end 31.43 21.27) (width 0.6) (layer "F.Cu") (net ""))
 (segment (start 79.69 69.53) (end 69.53 69.53) (width 0.6) (layer "F.Cu") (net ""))
 (segment (start 61.91 155.89) (end 64.45 155.89) (width 0.6) (layer "F.Cu") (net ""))
 (segment (start 41.59 160.97) (end 59.37 160.97) (width 0.6) (layer "F.Cu") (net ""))
 (segment (start 21.27 26.35) (end 46.67 26.35) (width 0.6) (layer "F.Cu") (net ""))
 (segment (start 39.05 155.89) (end 36.51 155.89) (width 0.6) (layer "F.Cu") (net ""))
 (segment (start 44.13 120.33) (end 36.51 89.85) (width 0.6) (layer "F.Cu") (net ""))
 (segment (start 39.05 36.51) (end 64.45 36.51) (width 0.6) (layer "F.Cu") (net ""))
 (segment (start 77.15 82.23) (end 28.89 82.23) (width 0.6) (layer "F.Cu") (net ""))
 (segment (start 69.53 160.97) (end 79.69 160.97) (width 0.6) (layer "F.Cu") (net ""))
 (segment (start 61.91 26.35) (end 66.989999 26.35) (width 0.6) (layer "F.Cu") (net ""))
 (segment (start 74.61 51.75) (end 41.59 51.75) (width 0.6) (layer "F.Cu") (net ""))
 (segment (start 31.43 160.97) (end 41.59 160.97) (width 0.6) (layer "F.Cu") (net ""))
 (segment (start 56.83 120.33) (end 41.59 120.33) (width 0.6) (layer "F.Cu") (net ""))
 (segment (start 39.05 26.35) (end 54.29 26.35) (width 0.6) (layer "F.Cu") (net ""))
 (segment (start 31.43 21.27) (end 41.59 21.27) (width 0.6) (layer "F.Cu") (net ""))
 (segment (start 51.75 140.65) (end 66.989999 140.65) (width 0.6) (layer "F.Cu") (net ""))
 (segment (start 49.21 140.65) (end 33.97 140.65) (width 0.6) (layer "F.Cu") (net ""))
 (segment (start 59.37 160.97) (end 69.53 160.97) (width 0.6) (layer "F.Cu") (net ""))
 (segment (start 21.27 160.97) (end 31.43 160.97) (width 0.6) (layer "F.Cu") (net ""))
 (segment (start 41.59 21.27) (end 51.75 21.27) (width 0.6) (layer "F.Cu") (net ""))
 (segment (start 51.75 21.27) (end 69.53 21.27) (width 0.6) (layer "F.Cu") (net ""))
 (segment (start 61.91 21.27) (end 61.91 28.89) (width 1.9) (layer "B.Cu") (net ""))
 (segment (start 39.05 33.97) (end 39.05 46.67) (width 1.9) (layer "B.Cu") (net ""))
 (segment (start 61.91 107.63) (end 61.91 148.27) (width 1.9) (layer "B.Cu") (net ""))
 (segment (start 77.15 66.989999) (end 77.15 77.15) (width 1.9) (layer "B.Cu") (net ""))
 (segment (start 46.67 107.63) (end 46.67 160.97) (width 1.9) (layer "B.Cu") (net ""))
 (segment (start 69.53 107.63) (end 69.53 160.97) (width 1.9) (layer "B.Cu") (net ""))
 (segment (start 61.91 33.97) (end 61.91 102.55) (width 1.9) (layer "B.Cu") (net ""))
 (segment (start 66.989999 107.63) (end 66.989999 160.97) (width 1.9) (layer "B.Cu") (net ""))
 (segment (start 46.67 21.27) (end 46.67 102.55) (width 1.9) (layer "B.Cu") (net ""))
 (segment (start 39.05 21.27) (end 39.05 28.89) (width 1.9) (layer "B.Cu") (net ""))
 (segment (start 54.29 107.63) (end 54.29 160.97) (width 1.9) (layer "B.Cu") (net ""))
 (segment (start 39.05 107.63) (end 39.05 148.27) (width 1.9) (layer "B.Cu") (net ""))
 (segment (start 31.43 21.27) (end 31.43 102.55) (width 1.9) (layer "B.Cu") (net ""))
 (segment (start 66.989999 21.27) (end 66.989999 102.55) (width 1.9) (layer "B.Cu") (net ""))
 (segment (start 59.37 107.63) (end 59.37 138.11) (width 1.9) (layer "B.Cu") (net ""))
 (segment (start 79.69 69.53) (end 79.69 72.07) (width 1.9) (layer "B.Cu") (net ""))
 (segment (start 41.59 21.27) (end 41.59 46.67) (width 1.9) (layer "B.Cu") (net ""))
 (segment (start 28.89 51.75) (end 28.89 102.55) (width 1.9) (layer "B.Cu") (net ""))
 (segment (start 77.15 92.39) (end 77.15 160.97) (width 1.9) (layer "B.Cu") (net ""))
 (segment (start 59.37 143.19) (end 59.37 160.97) (width 1.9) (layer "B.Cu") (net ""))
 (segment (start 79.69 77.15) (end 79.69 110.17) (width 1.9) (layer "B.Cu") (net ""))
 (segment (start 77.15 21.27) (end 77.15 61.91) (width 1.9) (layer "B.Cu") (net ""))
 (segment (start 41.59 51.75) (end 41.59 102.55) (width 1.9) (layer "B.Cu") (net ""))
 (segment (start 44.13 21.27) (end 44.13 102.55) (width 1.9) (layer "B.Cu") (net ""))
 (segment (start 61.91 153.35) (end 61.91 160.97) (width 1.9) (layer "B.Cu") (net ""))
 (segment (start 39.05 153.35) (end 39.05 160.97) (width 1.9) (layer "B.Cu") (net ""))
 (segment (start 49.21 21.27) (end 49.21 102.55) (width 1.9) (layer "B.Cu") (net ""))
 (segment (start 56.83 21.27) (end 56.83 102.55) (width 1.9) (layer "B.Cu") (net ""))
 (segment (start 36.51 21.27) (end 36.51 102.55) (width 1.9) (layer "B.Cu") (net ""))
 (segment (start 51.75 21.27) (end 51.75 46.67) (width 1.9) (layer "B.Cu") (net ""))
 (segment (start 49.21 107.63) (end 49.21 135.57) (width 1.9) (layer "B.Cu") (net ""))
 (segment (start 79.69 21.27) (end 79.69 33.97) (width 1.9) (layer "B.Cu") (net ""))
 (segment (start 56.83 107.63) (end 56.83 115.25) (width 1.9) (layer "B.Cu") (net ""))
 (segment (start 54.29 21.27) (end 54.29 102.55) (width 1.9) (layer "B.Cu") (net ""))
 (segment (start 74.61 21.27) (end 74.61 87.31) (width 1.9) (layer "B.Cu") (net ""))
 (segment (start 41.59 107.63) (end 41.59 130.49) (width 1.9) (layer "B.Cu") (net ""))
 (segment (start 21.27 21.27) (end 21.27 127.95) (width 1.9) (layer "B.Cu") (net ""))
 (segment (start 49.21 140.65) (end 49.21 160.97) (width 1.9) (layer "B.Cu") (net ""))
 (segment (start 26.35 21.27) (end 26.35 102.55) (width 1.9) (layer "B.Cu") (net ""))
 (segment (start 23.81 21.27) (end 23.81 160.97) (width 1.9) (layer "B.Cu") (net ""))
 (segment (start 74.61 92.39) (end 74.61 102.55) (width 1.9) (layer "B.Cu") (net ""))
 (segment (start 51.75 51.75) (end 51.75 102.55) (width 1.9) (layer "B.Cu") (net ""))
 (segment (start 31.43 107.63) (end 31.43 160.97) (width 1.9) (layer "B.Cu") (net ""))
 (segment (start 74.61 107.63) (end 74.61 160.97) (width 1.9) (layer "B.Cu") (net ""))
 (segment (start 79.69 39.05) (end 79.69 64.45) (width 1.9) (layer "B.Cu") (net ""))
 (segment (start 56.83 120.33) (end 56.83 160.97) (width 1.9) (layer "B.Cu") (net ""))
 (segment (start 64.45 107.63) (end 64.45 160.97) (width 1.9) (layer "B.Cu") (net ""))
 (segment (start 33.97 107.63) (end 33.97 160.97) (width 1.9) (layer "B.Cu") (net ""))
 (segment (start 79.69 115.25) (end 79.69 160.97) (width 1.9) (layer "B.Cu") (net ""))
 (segment (start 28.89 21.27) (end 28.89 46.67) (width 1.9) (layer "B.Cu") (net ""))
 (segment (start 64.45 21.27) (end 64.45 102.55) (width 1.9) (layer "B.Cu") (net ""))
 (segment (start 39.05 51.75) (end 39.05 102.55) (width 1.9) (layer "B.Cu") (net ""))
 (segment (start 59.37 21.27) (end 59.37 102.55) (width 1.9) (layer "B.Cu") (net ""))
 (segment (start 51.75 140.65) (end 51.75 160.97) (width 1.9) (layer "B.Cu") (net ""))
 (segment (start 26.35 107.63) (end 26.35 160.97) (width 1.9) (layer "B.Cu") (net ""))
 (segment (start 36.51 107.63) (end 36.51 160.97) (width 1.9) (layer "B.Cu") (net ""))
 (segment (start 69.53 21.27) (end 69.53 102.55) (width 1.9) (layer "B.Cu") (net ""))
 (segment (start 21.27 133.03) (end 21.27 160.97) (width 1.9) (layer "B.Cu") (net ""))
 (segment (start 44.13 120.33) (end 44.13 160.97) (width 1.9) (layer "B.Cu") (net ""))
 (segment (start 51.75 107.63) (end 51.75 135.57) (width 1.9) (layer "B.Cu") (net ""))
 (segment (start 77.15 82.23) (end 77.15 87.31) (width 1.9) (layer "B.Cu") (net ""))
 (segment (start 28.89 107.63) (end 28.89 160.97) (width 1.9) (layer "B.Cu") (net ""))
 (segment (start 41.59 135.57) (end 41.59 160.97) (width 1.9) (layer "B.Cu") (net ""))
 (segment (start 72.07 21.27) (end 72.07 102.55) (width 1.9) (layer "B.Cu") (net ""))
 (segment (start 72.07 107.63) (end 72.07 160.97) (width 1.9) (layer "B.Cu") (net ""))
 (segment (start 33.97 21.27) (end 33.97 102.55) (width 1.9) (layer "B.Cu") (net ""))
 (segment (start 44.13 107.63) (end 44.13 115.25) (width 1.9) (layer "B.Cu") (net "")))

